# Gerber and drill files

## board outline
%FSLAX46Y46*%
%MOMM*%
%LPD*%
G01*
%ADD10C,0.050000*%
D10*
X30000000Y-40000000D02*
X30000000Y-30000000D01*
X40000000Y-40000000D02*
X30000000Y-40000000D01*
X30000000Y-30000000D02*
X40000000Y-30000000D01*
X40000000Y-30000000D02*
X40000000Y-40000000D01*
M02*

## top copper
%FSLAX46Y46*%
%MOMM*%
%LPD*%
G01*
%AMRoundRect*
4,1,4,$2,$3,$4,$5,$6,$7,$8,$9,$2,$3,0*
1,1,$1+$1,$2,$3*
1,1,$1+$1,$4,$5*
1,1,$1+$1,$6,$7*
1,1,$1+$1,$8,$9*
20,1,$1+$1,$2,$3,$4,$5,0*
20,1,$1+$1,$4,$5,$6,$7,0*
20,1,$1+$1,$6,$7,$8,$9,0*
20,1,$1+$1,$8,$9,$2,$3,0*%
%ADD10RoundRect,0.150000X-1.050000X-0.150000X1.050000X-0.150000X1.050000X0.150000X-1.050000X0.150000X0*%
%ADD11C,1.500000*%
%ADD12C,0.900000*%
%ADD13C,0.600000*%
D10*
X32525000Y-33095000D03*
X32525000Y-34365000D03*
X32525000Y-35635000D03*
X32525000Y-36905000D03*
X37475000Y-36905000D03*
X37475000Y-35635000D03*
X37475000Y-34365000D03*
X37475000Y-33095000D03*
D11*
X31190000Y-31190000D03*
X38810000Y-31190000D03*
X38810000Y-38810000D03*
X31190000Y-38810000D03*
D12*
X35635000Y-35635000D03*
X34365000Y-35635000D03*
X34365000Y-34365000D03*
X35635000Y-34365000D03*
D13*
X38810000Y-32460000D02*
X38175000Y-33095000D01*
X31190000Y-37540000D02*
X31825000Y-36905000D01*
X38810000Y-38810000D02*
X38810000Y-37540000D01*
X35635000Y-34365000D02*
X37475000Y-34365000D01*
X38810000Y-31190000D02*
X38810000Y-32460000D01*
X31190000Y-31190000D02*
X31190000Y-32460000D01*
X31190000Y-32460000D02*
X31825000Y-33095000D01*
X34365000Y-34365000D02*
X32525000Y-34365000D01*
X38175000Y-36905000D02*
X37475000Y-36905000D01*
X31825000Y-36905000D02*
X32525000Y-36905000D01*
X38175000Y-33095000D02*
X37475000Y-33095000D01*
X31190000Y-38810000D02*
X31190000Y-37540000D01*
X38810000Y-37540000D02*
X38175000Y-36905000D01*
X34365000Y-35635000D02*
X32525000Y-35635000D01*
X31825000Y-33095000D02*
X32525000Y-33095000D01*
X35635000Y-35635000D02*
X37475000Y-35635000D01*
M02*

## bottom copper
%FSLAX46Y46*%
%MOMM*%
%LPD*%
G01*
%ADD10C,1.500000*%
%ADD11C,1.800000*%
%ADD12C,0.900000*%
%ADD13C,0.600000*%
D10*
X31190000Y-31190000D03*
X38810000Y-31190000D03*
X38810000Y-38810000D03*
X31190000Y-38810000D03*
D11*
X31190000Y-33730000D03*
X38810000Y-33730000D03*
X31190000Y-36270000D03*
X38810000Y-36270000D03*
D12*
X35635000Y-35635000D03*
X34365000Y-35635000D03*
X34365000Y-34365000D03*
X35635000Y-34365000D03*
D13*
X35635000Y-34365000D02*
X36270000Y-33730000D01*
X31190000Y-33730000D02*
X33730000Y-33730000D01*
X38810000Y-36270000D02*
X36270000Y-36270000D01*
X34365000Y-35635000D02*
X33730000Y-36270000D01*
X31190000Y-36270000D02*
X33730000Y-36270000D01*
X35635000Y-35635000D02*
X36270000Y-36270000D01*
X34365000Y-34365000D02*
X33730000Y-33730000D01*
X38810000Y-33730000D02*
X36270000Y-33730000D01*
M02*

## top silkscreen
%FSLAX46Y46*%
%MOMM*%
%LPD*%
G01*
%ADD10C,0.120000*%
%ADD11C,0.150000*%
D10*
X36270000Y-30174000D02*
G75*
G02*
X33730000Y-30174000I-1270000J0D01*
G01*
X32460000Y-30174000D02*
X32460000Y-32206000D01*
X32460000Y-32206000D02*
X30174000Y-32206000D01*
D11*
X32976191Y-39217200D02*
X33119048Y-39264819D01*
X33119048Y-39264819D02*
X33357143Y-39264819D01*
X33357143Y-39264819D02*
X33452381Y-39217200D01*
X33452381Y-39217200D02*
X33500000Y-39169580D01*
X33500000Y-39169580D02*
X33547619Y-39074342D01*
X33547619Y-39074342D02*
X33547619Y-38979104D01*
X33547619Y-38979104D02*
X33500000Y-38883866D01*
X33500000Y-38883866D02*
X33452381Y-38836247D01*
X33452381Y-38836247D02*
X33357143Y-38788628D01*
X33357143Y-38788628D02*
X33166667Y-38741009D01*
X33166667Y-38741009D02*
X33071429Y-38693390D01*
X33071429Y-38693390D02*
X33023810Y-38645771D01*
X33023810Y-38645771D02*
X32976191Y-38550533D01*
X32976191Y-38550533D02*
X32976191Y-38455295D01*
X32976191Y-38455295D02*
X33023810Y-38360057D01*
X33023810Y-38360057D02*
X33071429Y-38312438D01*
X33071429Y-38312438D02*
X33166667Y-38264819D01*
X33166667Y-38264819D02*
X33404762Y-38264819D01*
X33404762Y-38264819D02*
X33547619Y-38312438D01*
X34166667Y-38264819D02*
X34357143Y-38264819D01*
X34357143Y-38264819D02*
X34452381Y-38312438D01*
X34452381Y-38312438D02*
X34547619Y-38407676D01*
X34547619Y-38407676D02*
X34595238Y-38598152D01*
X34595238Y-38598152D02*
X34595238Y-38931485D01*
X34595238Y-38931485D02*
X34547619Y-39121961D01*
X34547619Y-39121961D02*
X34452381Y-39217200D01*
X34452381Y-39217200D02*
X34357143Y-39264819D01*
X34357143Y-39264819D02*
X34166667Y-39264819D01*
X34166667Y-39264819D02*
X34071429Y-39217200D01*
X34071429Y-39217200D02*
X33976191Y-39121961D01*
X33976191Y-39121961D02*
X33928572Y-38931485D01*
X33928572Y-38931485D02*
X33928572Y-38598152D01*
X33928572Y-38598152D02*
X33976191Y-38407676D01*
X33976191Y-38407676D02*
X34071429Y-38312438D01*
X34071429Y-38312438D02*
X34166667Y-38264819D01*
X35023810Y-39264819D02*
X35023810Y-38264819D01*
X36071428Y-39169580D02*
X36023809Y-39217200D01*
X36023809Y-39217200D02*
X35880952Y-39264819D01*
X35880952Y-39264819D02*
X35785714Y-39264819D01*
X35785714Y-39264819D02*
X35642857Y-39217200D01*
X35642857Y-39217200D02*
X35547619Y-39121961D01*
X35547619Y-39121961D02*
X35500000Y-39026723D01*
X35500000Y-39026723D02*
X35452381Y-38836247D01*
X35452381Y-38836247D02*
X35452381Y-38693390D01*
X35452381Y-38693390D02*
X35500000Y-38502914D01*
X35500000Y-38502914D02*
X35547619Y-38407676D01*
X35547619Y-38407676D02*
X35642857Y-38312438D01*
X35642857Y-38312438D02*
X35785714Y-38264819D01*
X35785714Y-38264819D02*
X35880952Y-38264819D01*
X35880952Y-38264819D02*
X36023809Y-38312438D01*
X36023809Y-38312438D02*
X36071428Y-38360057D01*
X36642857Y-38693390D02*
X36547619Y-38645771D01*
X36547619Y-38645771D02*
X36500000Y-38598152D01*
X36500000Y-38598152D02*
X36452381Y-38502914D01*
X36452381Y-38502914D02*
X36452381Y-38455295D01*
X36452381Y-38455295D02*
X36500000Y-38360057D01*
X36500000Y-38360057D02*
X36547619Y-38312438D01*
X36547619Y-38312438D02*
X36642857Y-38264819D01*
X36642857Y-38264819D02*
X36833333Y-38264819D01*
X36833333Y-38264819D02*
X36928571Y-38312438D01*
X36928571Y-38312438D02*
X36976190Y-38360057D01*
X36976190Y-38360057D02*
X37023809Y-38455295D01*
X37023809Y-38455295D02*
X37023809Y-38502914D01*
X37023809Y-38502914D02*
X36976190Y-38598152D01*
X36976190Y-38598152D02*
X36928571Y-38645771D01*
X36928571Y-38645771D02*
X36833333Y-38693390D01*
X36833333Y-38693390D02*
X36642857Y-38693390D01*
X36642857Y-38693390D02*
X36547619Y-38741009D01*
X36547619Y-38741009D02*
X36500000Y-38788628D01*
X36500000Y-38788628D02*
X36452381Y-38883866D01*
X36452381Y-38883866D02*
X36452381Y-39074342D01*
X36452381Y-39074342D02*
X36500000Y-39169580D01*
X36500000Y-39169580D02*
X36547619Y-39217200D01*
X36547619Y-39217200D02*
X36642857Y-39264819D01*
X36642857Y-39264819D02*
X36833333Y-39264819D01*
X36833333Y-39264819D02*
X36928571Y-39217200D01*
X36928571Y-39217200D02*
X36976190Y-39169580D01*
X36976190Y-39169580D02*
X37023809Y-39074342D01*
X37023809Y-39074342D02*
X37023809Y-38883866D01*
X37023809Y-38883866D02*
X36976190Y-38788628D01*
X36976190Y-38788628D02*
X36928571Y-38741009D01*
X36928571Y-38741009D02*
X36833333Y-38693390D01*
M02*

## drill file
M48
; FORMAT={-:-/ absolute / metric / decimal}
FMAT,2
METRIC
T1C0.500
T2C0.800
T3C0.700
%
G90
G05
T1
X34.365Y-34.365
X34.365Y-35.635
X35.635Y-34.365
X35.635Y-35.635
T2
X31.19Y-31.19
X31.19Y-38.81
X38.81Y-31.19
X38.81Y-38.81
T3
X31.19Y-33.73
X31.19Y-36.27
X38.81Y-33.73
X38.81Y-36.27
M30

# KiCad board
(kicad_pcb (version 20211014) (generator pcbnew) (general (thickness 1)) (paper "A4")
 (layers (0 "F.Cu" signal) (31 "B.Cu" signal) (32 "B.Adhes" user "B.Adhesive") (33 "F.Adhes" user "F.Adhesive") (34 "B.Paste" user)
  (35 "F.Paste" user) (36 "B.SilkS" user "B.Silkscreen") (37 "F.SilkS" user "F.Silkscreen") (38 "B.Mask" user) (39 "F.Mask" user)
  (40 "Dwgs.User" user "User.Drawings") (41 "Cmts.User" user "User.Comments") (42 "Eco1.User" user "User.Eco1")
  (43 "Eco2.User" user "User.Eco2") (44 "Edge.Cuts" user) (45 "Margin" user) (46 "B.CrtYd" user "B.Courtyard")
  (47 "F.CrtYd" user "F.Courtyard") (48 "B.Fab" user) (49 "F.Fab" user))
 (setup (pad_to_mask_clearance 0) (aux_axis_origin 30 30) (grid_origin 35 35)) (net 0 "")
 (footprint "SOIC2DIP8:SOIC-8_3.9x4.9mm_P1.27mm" (layer "F.Cu") (at 35 35)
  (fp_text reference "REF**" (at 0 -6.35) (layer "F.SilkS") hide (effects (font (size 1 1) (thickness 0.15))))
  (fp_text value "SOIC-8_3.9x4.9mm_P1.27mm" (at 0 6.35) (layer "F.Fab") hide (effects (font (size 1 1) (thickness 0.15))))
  (pad "1" smd roundrect locked (at -2.475 -1.905) (size 2.4 0.6) (layers "F.Cu" "F.Paste" "F.Mask") (roundrect_rratio 0.25))
  (pad "2" smd roundrect locked (at -2.475 -0.635) (size 2.4 0.6) (layers "F.Cu" "F.Paste" "F.Mask") (roundrect_rratio 0.25))
  (pad "3" smd roundrect locked (at -2.475 0.635) (size 2.4 0.6) (layers "F.Cu" "F.Paste" "F.Mask") (roundrect_rratio 0.25))
  (pad "4" smd roundrect locked (at -2.475 1.905) (size 2.4 0.6) (layers "F.Cu" "F.Paste" "F.Mask") (roundrect_rratio 0.25))
  (pad "5" smd roundrect locked (at 2.475 1.905) (size 2.4 0.6) (layers "F.Cu" "F.Paste" "F.Mask") (roundrect_rratio 0.25))
  (pad "6" smd roundrect locked (at 2.475 0.635) (size 2.4 0.6) (layers "F.Cu" "F.Paste" "F.Mask") (roundrect_rratio 0.25))
  (pad "7" smd roundrect locked (at 2.475 -0.635) (size 2.4 0.6) (layers "F.Cu" "F.Paste" "F.Mask") (roundrect_rratio 0.25))
  (pad "8" smd roundrect locked (at 2.475 -1.905) (size 2.4 0.6) (layers "F.Cu" "F.Paste" "F.Mask") (roundrect_rratio 0.25)))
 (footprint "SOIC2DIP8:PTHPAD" (layer "F.Cu") (at 31.19 31.19)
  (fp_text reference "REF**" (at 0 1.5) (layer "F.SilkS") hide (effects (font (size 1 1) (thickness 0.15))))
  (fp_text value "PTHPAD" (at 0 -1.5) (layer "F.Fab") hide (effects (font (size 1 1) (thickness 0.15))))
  (pad "1" thru_hole circle locked (at 0 0) (size 1.5 1.5) (drill 0.8) (layers *.Cu *.Mask)))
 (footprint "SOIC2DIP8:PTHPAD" (layer "F.Cu") (at 38.81 31.19)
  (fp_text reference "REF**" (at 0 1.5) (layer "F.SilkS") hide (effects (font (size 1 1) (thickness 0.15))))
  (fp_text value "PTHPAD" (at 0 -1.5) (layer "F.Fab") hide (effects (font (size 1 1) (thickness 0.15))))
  (pad "1" thru_hole circle locked (at 0 0) (size 1.5 1.5) (drill 0.8) (layers *.Cu *.Mask)))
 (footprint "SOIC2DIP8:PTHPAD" (layer "F.Cu") (at 38.81 38.81)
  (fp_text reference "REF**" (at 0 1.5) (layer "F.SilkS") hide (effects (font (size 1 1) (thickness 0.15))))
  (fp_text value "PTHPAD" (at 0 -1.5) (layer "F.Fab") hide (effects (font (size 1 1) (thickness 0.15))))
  (pad "1" thru_hole circle locked (at 0 0) (size 1.5 1.5) (drill 0.8) (layers *.Cu *.Mask)))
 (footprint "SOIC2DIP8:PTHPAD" (layer "F.Cu") (at 31.19 38.81)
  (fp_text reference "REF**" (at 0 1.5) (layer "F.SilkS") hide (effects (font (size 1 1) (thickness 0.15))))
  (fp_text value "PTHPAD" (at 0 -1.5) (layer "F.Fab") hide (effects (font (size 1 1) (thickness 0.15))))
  (pad "1" thru_hole circle locked (at 0 0) (size 1.5 1.5) (drill 0.8) (layers *.Cu *.Mask)))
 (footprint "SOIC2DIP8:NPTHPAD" (layer "F.Cu") (at 31.19 33.73)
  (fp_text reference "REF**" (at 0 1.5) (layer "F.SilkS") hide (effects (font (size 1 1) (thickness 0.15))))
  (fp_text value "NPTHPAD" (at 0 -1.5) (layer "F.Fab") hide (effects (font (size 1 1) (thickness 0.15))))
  (pad "" np_thru_hole circle (at 0 0) (size 1.8 1.8) (drill 0.7) (layers "B.Cu" "B.Mask")))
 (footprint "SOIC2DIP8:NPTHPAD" (layer "F.Cu") (at 38.81 33.73)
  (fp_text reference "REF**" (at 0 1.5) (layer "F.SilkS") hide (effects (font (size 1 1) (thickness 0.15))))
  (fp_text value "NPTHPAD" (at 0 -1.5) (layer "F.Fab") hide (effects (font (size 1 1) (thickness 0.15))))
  (pad "" np_thru_hole circle (at 0 0) (size 1.8 1.8) (drill 0.7) (layers "B.Cu" "B.Mask")))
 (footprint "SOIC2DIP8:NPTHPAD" (layer "F.Cu") (at 31.19 36.27)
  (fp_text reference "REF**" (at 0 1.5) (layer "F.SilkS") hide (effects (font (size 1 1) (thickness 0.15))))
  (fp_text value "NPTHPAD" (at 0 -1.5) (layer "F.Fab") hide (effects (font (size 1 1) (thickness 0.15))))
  (pad "" np_thru_hole circle (at 0 0) (size 1.8 1.8) (drill 0.7) (layers "B.Cu" "B.Mask")))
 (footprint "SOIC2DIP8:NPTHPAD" (layer "F.Cu") (at 38.81 36.27)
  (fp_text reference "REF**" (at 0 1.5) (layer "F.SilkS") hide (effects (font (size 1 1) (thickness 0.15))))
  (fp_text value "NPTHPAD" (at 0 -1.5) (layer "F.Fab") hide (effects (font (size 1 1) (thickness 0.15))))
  (pad "" np_thru_hole circle (at 0 0) (size 1.8 1.8) (drill 0.7) (layers "B.Cu" "B.Mask")))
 (gr_arc (start 36.27 30.174) (mid 35 31.444) (end 33.73 30.174) (layer "F.SilkS") (width 0.12))
 (gr_line (start 32.46 30.174) (end 32.46 32.206) (layer "F.SilkS") (width 0.12))
 (gr_line (start 32.46 32.206) (end 30.174 32.206) (layer "F.SilkS") (width 0.12))
 (gr_line (start 30 40) (end 30 30) (layer "Edge.Cuts") (width 0.05))
 (gr_line (start 40 40) (end 30 40) (layer "Edge.Cuts") (width 0.05))
 (gr_line (start 30 30) (end 40 30) (layer "Edge.Cuts") (width 0.05))
 (gr_line (start 40 30) (end 40 40) (layer "Edge.Cuts") (width 0.05))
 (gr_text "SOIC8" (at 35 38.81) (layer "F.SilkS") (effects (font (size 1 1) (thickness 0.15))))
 (segment (start 38.81 32.46) (end 38.175 33.095) (width 0.6) (layer "F.Cu") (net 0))
 (segment (start 31.19 37.54) (end 31.825 36.905) (width 0.6) (layer "F.Cu") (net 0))
 (segment (start 38.81 38.81) (end 38.81 37.54) (width 0.6) (layer "F.Cu") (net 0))
 (segment (start 35.635 34.365) (end 37.475 34.365) (width 0.6) (layer "F.Cu") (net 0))
 (segment (start 38.81 31.19) (end 38.81 32.46) (width 0.6) (layer "F.Cu") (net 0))
 (segment (start 31.19 31.19) (end 31.19 32.46) (width 0.6) (layer "F.Cu") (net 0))
 (segment (start 31.19 32.46) (end 31.825 33.095) (width 0.6) (layer "F.Cu") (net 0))
 (segment (start 34.365 34.365) (end 32.525 34.365) (width 0.6) (layer "F.Cu") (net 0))
 (segment (start 38.175 36.905) (end 37.475 36.905) (width 0.6) (layer "F.Cu") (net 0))
 (segment (start 31.825 36.905) (end 32.525 36.905) (width 0.6) (layer "F.Cu") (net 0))
 (segment (start 38.175 33.095) (end 37.475 33.095) (width 0.6) (layer "F.Cu") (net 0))
 (segment (start 31.19 38.81) (end 31.19 37.54) (width 0.6) (layer "F.Cu") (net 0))
 (segment (start 38.81 37.54) (end 38.175 36.905) (width 0.6) (layer "F.Cu") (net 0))
 (segment (start 34.365 35.635) (end 32.525 35.635) (width 0.6) (layer "F.Cu") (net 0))
 (segment (start 31.825 33.095) (end 32.525 33.095) (width 0.6) (layer "F.Cu") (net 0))
 (segment (start 35.635 35.635) (end 37.475 35.635) (width 0.6) (layer "F.Cu") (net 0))
 (via (at 35.635 35.635) (size 0.9) (drill 0.5) (layers "F.Cu" "B.Cu") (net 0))
 (via (at 34.365 35.635) (size 0.9) (drill 0.5) (layers "F.Cu" "B.Cu") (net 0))
 (via (at 34.365 34.365) (size 0.9) (drill 0.5) (layers "F.Cu" "B.Cu") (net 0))
 (via (at 35.635 34.365) (size 0.9) (drill 0.5) (layers "F.Cu" "B.Cu") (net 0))
 (segment (start 35.635 34.365) (end 36.27 33.73) (width 0.6) (layer "B.Cu") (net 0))
 (segment (start 31.19 33.73) (end 33.73 33.73) (width 0.6) (layer "B.Cu") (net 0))
 (segment (start 38.81 36.27) (end 36.27 36.27) (width 0.6) (layer "B.Cu") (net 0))
 (segment (start 34.365 35.635) (end 33.73 36.27) (width 0.6) (layer "B.Cu") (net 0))
 (segment (start 31.19 36.27) (end 33.73 36.27) (width 0.6) (layer "B.Cu") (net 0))
 (segment (start 35.635 35.635) (end 36.27 36.27) (width 0.6) (layer "B.Cu") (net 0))
 (segment (start 34.365 34.365) (end 33.73 33.73) (width 0.6) (layer "B.Cu") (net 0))
 (segment (start 38.81 33.73) (end 36.27 33.73) (width 0.6) (layer "B.Cu") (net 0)))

